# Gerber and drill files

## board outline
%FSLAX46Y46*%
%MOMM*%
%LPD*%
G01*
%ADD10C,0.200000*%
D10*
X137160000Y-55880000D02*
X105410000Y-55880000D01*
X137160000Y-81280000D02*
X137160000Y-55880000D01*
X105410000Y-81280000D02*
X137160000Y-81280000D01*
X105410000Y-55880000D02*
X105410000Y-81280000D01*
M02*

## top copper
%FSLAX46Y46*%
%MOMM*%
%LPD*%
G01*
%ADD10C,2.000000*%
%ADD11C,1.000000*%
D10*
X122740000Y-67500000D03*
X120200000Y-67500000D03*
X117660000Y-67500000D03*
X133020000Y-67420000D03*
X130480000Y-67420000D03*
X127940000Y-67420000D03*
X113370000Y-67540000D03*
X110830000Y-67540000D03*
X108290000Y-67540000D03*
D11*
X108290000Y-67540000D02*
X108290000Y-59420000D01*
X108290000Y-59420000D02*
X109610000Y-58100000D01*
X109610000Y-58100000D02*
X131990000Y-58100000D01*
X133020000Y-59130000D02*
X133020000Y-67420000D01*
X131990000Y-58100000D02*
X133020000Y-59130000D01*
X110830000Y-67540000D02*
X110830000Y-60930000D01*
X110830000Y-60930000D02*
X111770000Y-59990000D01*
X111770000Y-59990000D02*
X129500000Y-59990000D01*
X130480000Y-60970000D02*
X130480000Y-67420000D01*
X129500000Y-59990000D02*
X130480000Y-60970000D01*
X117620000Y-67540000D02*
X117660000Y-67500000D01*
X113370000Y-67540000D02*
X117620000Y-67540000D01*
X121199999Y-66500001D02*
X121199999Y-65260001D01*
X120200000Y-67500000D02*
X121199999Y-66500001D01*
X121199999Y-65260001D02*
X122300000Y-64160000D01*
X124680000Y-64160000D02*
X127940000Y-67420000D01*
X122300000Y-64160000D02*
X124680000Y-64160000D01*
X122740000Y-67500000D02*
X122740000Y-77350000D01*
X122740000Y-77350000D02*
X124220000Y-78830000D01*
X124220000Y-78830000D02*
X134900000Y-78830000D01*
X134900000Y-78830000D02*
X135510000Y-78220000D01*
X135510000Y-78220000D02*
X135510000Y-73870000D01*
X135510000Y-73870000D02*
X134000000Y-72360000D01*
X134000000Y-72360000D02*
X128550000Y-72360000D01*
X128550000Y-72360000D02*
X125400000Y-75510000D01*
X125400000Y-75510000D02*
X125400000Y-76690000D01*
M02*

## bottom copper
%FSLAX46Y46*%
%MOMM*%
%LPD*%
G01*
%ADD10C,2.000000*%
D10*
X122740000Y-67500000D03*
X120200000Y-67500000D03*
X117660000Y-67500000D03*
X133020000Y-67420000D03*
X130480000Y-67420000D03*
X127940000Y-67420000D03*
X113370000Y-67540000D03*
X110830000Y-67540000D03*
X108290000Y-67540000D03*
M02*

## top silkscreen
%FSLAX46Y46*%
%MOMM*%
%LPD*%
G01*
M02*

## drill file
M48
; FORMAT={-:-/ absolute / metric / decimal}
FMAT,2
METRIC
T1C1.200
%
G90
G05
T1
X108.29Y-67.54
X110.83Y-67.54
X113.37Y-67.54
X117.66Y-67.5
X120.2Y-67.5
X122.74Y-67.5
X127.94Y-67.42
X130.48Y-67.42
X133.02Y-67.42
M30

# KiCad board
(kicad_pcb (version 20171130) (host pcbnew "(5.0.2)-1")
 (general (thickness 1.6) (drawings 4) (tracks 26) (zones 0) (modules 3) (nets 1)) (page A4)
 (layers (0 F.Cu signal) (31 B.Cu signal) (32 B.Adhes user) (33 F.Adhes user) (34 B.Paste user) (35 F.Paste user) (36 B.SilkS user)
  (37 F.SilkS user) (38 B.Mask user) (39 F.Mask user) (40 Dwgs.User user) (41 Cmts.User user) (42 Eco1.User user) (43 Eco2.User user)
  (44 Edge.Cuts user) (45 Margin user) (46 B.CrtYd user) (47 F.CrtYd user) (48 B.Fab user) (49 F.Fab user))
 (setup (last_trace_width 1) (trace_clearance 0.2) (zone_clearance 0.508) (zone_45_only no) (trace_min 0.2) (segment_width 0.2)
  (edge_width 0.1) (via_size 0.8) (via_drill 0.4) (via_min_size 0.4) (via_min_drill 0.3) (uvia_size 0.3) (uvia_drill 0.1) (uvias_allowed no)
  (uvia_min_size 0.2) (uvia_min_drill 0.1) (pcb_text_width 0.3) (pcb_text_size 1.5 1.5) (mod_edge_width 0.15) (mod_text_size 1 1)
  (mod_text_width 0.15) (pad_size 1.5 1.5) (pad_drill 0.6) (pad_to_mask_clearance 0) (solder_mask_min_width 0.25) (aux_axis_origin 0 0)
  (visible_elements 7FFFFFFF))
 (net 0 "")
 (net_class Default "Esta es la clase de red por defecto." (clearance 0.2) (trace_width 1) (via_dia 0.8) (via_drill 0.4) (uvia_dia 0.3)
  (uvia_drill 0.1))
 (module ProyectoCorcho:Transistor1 (layer F.Cu) (at 120.2 67.5)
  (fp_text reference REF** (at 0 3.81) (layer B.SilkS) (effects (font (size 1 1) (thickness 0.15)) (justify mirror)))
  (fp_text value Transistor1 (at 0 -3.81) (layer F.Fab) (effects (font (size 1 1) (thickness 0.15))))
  (pad 3 thru_hole circle (at 2.54 0) (size 2 2) (drill 1.2) (layers *.Cu *.Mask))
  (pad 2 thru_hole circle (at 0 0) (size 2 2) (drill 1.2) (layers *.Cu *.Mask))
  (pad 1 thru_hole circle (at -2.54 0) (size 2 2) (drill 1.2) (layers *.Cu *.Mask)))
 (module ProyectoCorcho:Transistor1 (layer F.Cu) (at 130.48 67.42)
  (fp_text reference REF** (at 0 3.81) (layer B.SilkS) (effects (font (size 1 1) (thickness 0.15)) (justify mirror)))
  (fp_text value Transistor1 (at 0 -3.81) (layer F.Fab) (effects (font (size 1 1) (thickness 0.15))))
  (pad 3 thru_hole circle (at 2.54 0) (size 2 2) (drill 1.2) (layers *.Cu *.Mask))
  (pad 2 thru_hole circle (at 0 0) (size 2 2) (drill 1.2) (layers *.Cu *.Mask))
  (pad 1 thru_hole circle (at -2.54 0) (size 2 2) (drill 1.2) (layers *.Cu *.Mask)))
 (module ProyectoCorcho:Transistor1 (layer F.Cu) (at 110.83 67.54)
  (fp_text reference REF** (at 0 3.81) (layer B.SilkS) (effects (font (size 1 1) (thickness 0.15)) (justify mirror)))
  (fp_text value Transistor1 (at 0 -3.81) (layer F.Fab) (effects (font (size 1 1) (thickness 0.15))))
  (pad 3 thru_hole circle (at 2.54 0) (size 2 2) (drill 1.2) (layers *.Cu *.Mask))
  (pad 2 thru_hole circle (at 0 0) (size 2 2) (drill 1.2) (layers *.Cu *.Mask))
  (pad 1 thru_hole circle (at -2.54 0) (size 2 2) (drill 1.2) (layers *.Cu *.Mask)))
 (gr_line (start 137.16 55.88) (end 105.41 55.88) (layer Edge.Cuts) (width 0.2))
 (gr_line (start 137.16 81.28) (end 137.16 55.88) (layer Edge.Cuts) (width 0.2))
 (gr_line (start 105.41 81.28) (end 137.16 81.28) (layer Edge.Cuts) (width 0.2))
 (gr_line (start 105.41 55.88) (end 105.41 81.28) (layer Edge.Cuts) (width 0.2))
 (segment (start 108.29 67.54) (end 108.29 59.42) (width 1) (layer F.Cu) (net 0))
 (segment (start 108.29 59.42) (end 109.61 58.1) (width 1) (layer F.Cu) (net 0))
 (segment (start 109.61 58.1) (end 131.99 58.1) (width 1) (layer F.Cu) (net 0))
 (segment (start 133.02 59.13) (end 133.02 67.42) (width 1) (layer F.Cu) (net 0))
 (segment (start 131.99 58.1) (end 133.02 59.13) (width 1) (layer F.Cu) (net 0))
 (segment (start 110.83 67.54) (end 110.83 60.93) (width 1) (layer F.Cu) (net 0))
 (segment (start 110.83 60.93) (end 111.77 59.99) (width 1) (layer F.Cu) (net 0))
 (segment (start 111.77 59.99) (end 129.5 59.99) (width 1) (layer F.Cu) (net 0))
 (segment (start 130.48 60.97) (end 130.48 67.42) (width 1) (layer F.Cu) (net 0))
 (segment (start 129.5 59.99) (end 130.48 60.97) (width 1) (layer F.Cu) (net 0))
 (segment (start 117.62 67.54) (end 117.66 67.5) (width 1) (layer F.Cu) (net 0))
 (segment (start 113.37 67.54) (end 117.62 67.54) (width 1) (layer F.Cu) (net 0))
 (segment (start 121.199999 66.500001) (end 121.199999 65.260001) (width 1) (layer F.Cu) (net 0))
 (segment (start 120.2 67.5) (end 121.199999 66.500001) (width 1) (layer F.Cu) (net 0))
 (segment (start 121.199999 65.260001) (end 122.3 64.16) (width 1) (layer F.Cu) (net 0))
 (segment (start 124.68 64.16) (end 127.94 67.42) (width 1) (layer F.Cu) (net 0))
 (segment (start 122.3 64.16) (end 124.68 64.16) (width 1) (layer F.Cu) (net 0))
 (segment (start 122.74 67.5) (end 122.74 77.35) (width 1) (layer F.Cu) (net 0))
 (segment (start 122.74 77.35) (end 124.22 78.83) (width 1) (layer F.Cu) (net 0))
 (segment (start 124.22 78.83) (end 134.9 78.83) (width 1) (layer F.Cu) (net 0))
 (segment (start 134.9 78.83) (end 135.51 78.22) (width 1) (layer F.Cu) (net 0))
 (segment (start 135.51 78.22) (end 135.51 73.87) (width 1) (layer F.Cu) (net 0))
 (segment (start 135.51 73.87) (end 134 72.36) (width 1) (layer F.Cu) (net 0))
 (segment (start 134 72.36) (end 128.55 72.36) (width 1) (layer F.Cu) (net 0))
 (segment (start 128.55 72.36) (end 125.4 75.51) (width 1) (layer F.Cu) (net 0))
 (segment (start 125.4 75.51) (end 125.4 76.69) (width 1) (layer F.Cu) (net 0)))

